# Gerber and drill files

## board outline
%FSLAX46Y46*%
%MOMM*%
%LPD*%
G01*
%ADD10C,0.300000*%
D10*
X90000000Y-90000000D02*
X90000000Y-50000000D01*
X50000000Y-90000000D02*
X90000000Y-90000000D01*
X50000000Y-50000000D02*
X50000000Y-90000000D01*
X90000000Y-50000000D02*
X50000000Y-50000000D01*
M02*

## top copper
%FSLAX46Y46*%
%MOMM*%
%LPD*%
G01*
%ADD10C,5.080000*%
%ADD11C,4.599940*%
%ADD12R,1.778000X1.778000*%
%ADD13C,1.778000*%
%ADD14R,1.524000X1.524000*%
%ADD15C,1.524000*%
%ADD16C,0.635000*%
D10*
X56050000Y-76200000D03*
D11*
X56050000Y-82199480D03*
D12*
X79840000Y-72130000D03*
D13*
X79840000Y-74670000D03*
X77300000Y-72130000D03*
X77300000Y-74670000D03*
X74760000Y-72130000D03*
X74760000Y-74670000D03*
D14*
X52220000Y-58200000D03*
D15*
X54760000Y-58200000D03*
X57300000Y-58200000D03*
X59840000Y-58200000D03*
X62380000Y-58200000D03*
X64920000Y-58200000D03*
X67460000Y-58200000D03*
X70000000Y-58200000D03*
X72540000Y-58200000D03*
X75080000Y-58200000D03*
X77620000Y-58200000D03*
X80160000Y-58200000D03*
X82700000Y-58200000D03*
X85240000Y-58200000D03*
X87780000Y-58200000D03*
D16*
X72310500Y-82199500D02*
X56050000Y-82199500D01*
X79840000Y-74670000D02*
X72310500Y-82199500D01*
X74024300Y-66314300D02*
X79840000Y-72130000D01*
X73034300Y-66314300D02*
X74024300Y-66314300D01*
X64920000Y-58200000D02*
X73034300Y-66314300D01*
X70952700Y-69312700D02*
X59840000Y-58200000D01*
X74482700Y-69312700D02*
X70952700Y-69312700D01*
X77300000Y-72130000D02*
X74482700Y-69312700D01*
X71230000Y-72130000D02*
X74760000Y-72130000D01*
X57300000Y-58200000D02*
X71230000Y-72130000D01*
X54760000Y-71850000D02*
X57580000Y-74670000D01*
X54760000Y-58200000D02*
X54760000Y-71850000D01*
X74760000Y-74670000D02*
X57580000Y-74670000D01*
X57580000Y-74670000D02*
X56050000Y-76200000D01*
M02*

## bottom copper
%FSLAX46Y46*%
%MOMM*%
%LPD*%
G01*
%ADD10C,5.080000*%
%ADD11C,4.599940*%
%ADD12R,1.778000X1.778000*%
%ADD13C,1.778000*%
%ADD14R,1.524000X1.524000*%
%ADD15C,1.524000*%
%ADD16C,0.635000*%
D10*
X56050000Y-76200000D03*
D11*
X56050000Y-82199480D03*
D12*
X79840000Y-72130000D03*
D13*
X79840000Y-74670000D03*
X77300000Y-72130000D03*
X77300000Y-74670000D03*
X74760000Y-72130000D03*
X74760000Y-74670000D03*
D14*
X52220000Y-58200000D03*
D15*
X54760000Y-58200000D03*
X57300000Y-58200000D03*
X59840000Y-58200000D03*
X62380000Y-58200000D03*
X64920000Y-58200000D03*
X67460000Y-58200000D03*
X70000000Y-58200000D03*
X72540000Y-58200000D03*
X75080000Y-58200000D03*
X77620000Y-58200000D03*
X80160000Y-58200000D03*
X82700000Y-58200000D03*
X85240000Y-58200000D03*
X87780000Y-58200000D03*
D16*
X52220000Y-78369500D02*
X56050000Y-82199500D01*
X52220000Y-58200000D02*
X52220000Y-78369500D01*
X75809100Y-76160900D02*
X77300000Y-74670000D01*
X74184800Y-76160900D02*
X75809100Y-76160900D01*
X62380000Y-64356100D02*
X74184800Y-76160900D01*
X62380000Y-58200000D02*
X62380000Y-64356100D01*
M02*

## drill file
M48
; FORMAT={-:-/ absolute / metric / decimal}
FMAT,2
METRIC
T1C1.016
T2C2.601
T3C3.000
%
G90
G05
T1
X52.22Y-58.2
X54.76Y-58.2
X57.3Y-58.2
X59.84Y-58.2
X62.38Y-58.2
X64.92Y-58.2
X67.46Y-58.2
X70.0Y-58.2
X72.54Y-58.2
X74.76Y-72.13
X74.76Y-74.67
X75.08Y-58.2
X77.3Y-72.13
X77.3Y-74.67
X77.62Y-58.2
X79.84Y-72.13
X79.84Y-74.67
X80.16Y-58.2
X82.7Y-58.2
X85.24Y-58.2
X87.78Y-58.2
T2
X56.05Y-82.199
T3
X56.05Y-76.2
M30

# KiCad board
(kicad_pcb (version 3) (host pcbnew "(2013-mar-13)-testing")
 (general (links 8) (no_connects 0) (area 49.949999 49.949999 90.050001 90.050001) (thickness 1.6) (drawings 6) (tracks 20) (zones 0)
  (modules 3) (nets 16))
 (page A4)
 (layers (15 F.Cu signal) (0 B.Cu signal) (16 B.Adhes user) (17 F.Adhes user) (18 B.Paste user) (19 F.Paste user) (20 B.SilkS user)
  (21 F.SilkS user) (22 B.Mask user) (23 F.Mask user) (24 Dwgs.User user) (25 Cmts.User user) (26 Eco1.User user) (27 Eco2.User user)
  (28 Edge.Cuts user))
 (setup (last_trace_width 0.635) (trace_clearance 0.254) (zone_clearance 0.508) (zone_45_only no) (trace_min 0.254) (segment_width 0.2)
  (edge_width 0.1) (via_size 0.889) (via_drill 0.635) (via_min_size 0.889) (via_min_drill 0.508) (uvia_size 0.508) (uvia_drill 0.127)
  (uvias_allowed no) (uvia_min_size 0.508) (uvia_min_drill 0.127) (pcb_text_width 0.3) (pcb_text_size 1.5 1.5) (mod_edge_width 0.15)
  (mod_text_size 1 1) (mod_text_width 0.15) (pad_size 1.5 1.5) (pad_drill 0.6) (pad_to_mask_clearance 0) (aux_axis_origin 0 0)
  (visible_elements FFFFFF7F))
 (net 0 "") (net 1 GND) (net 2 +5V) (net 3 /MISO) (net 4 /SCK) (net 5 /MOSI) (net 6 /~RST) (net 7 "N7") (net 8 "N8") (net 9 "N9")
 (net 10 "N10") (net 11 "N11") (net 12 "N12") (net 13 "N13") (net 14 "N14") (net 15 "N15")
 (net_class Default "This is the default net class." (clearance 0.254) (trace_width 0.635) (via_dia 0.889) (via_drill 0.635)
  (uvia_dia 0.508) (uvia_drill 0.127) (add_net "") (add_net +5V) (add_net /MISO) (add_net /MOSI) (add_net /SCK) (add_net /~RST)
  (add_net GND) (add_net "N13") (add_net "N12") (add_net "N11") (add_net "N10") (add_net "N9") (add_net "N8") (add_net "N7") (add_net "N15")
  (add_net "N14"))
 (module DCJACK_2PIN (layer F.Cu) (at 56.05 76.2 270)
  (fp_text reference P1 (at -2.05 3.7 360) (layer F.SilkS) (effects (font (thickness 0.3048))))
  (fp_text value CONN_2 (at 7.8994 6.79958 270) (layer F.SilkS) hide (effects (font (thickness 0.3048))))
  (pad 1 thru_hole circle (at 0 0 270) (size 5.08 5.08) (drill 2.99974) (layers *.Cu *.Mask F.SilkS) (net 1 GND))
  (pad 2 thru_hole circle (at 5.99948 0 270) (size 4.59994 4.59994) (drill 2.60096) (layers *.Cu *.Mask F.SilkS) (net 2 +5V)))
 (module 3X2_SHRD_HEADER (layer F.Cu) (at 77.3 73.4 180)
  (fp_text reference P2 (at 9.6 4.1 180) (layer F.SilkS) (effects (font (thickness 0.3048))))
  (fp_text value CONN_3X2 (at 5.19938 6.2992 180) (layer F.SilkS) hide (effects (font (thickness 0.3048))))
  (pad 1 thru_hole rect (at -2.54 1.27 180) (size 1.778 1.778) (drill 1.016) (layers *.Cu *.Mask F.SilkS) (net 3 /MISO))
  (pad 2 thru_hole circle (at -2.54 -1.27 180) (size 1.778 1.778) (drill 1.016) (layers *.Cu *.Mask F.SilkS) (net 2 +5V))
  (pad 3 thru_hole circle (at 0 1.27 180) (size 1.778 1.778) (drill 1.016) (layers *.Cu *.Mask F.SilkS) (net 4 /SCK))
  (pad 4 thru_hole circle (at 0 -1.27 180) (size 1.778 1.778) (drill 1.016) (layers *.Cu *.Mask F.SilkS) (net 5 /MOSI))
  (pad 5 thru_hole circle (at 2.54 1.27 180) (size 1.778 1.778) (drill 1.016) (layers *.Cu *.Mask F.SilkS) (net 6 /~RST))
  (pad 6 thru_hole circle (at 2.54 -1.27 180) (size 1.778 1.778) (drill 1.016) (layers *.Cu *.Mask F.SilkS) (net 1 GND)))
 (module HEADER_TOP (layer F.Cu) (at 70 58.2)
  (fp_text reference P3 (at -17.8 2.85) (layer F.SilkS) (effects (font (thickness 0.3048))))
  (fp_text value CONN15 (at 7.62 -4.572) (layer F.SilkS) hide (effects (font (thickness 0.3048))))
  (pad 1 thru_hole rect (at -17.78 0) (size 1.524 1.524) (drill 1.016) (layers *.Cu *.Mask F.SilkS) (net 2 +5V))
  (pad 2 thru_hole circle (at -15.24 0) (size 1.524 1.524) (drill 1.016) (layers *.Cu *.Mask F.SilkS) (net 1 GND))
  (pad 3 thru_hole circle (at -12.7 0) (size 1.524 1.524) (drill 1.016) (layers *.Cu *.Mask F.SilkS) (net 6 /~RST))
  (pad 4 thru_hole circle (at -10.16 0) (size 1.524 1.524) (drill 1.016) (layers *.Cu *.Mask F.SilkS) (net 4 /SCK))
  (pad 5 thru_hole circle (at -7.62 0) (size 1.524 1.524) (drill 1.016) (layers *.Cu *.Mask F.SilkS) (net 5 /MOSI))
  (pad 6 thru_hole circle (at -5.08 0) (size 1.524 1.524) (drill 1.016) (layers *.Cu *.Mask F.SilkS) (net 3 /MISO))
  (pad 7 thru_hole circle (at -2.54 0) (size 1.524 1.524) (drill 1.016) (layers *.Cu *.Mask F.SilkS) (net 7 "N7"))
  (pad 8 thru_hole circle (at 0 0) (size 1.524 1.524) (drill 1.016) (layers *.Cu *.Mask F.SilkS) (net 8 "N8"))
  (pad 9 thru_hole circle (at 2.54 0) (size 1.524 1.524) (drill 1.016) (layers *.Cu *.Mask F.SilkS) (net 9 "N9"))
  (pad 10 thru_hole circle (at 5.08 0) (size 1.524 1.524) (drill 1.016) (layers *.Cu *.Mask F.SilkS) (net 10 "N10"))
  (pad 11 thru_hole circle (at 7.62 0) (size 1.524 1.524) (drill 1.016) (layers *.Cu *.Mask F.SilkS) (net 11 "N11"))
  (pad 12 thru_hole circle (at 10.16 0) (size 1.524 1.524) (drill 1.016) (layers *.Cu *.Mask F.SilkS) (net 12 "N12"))
  (pad 13 thru_hole circle (at 12.7 0) (size 1.524 1.524) (drill 1.016) (layers *.Cu *.Mask F.SilkS) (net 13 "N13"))
  (pad 14 thru_hole circle (at 15.24 0) (size 1.524 1.524) (drill 1.016) (layers *.Cu *.Mask F.SilkS) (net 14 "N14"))
  (pad 15 thru_hole circle (at 17.78 0) (size 1.524 1.524) (drill 1.016) (layers *.Cu *.Mask F.SilkS) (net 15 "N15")))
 (gr_line (start 90 90) (end 90 50) (angle 90) (layer Edge.Cuts) (width 0.3))
 (gr_line (start 50 90) (end 90 90) (angle 90) (layer Edge.Cuts) (width 0.3))
 (gr_line (start 50 50) (end 50 90) (angle 90) (layer Edge.Cuts) (width 0.3))
 (gr_line (start 90 50) (end 50 50) (angle 90) (layer Edge.Cuts) (width 0.3))
 (segment (start 52.22 78.3695) (end 56.05 82.1995) (width 0.635) (layer B.Cu) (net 2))
 (segment (start 52.22 58.2) (end 52.22 78.3695) (width 0.635) (layer B.Cu) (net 2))
 (segment (start 72.3105 82.1995) (end 56.05 82.1995) (width 0.635) (layer F.Cu) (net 2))
 (segment (start 79.84 74.67) (end 72.3105 82.1995) (width 0.635) (layer F.Cu) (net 2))
 (segment (start 74.0243 66.3143) (end 79.84 72.13) (width 0.635) (layer F.Cu) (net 3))
 (segment (start 73.0343 66.3143) (end 74.0243 66.3143) (width 0.635) (layer F.Cu) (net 3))
 (segment (start 64.92 58.2) (end 73.0343 66.3143) (width 0.635) (layer F.Cu) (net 3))
 (segment (start 75.8091 76.1609) (end 77.3 74.67) (width 0.635) (layer B.Cu) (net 5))
 (segment (start 74.1848 76.1609) (end 75.8091 76.1609) (width 0.635) (layer B.Cu) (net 5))
 (segment (start 62.38 64.3561) (end 74.1848 76.1609) (width 0.635) (layer B.Cu) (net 5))
 (segment (start 62.38 58.2) (end 62.38 64.3561) (width 0.635) (layer B.Cu) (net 5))
 (segment (start 70.9527 69.3127) (end 59.84 58.2) (width 0.635) (layer F.Cu) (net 4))
 (segment (start 74.4827 69.3127) (end 70.9527 69.3127) (width 0.635) (layer F.Cu) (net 4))
 (segment (start 77.3 72.13) (end 74.4827 69.3127) (width 0.635) (layer F.Cu) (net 4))
 (segment (start 71.23 72.13) (end 74.76 72.13) (width 0.635) (layer F.Cu) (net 6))
 (segment (start 57.3 58.2) (end 71.23 72.13) (width 0.635) (layer F.Cu) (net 6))
 (segment (start 54.76 71.85) (end 57.58 74.67) (width 0.635) (layer F.Cu) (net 1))
 (segment (start 54.76 58.2) (end 54.76 71.85) (width 0.635) (layer F.Cu) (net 1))
 (segment (start 74.76 74.67) (end 57.58 74.67) (width 0.635) (layer F.Cu) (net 1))
 (segment (start 57.58 74.67) (end 56.05 76.2) (width 0.635) (layer F.Cu) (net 1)))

